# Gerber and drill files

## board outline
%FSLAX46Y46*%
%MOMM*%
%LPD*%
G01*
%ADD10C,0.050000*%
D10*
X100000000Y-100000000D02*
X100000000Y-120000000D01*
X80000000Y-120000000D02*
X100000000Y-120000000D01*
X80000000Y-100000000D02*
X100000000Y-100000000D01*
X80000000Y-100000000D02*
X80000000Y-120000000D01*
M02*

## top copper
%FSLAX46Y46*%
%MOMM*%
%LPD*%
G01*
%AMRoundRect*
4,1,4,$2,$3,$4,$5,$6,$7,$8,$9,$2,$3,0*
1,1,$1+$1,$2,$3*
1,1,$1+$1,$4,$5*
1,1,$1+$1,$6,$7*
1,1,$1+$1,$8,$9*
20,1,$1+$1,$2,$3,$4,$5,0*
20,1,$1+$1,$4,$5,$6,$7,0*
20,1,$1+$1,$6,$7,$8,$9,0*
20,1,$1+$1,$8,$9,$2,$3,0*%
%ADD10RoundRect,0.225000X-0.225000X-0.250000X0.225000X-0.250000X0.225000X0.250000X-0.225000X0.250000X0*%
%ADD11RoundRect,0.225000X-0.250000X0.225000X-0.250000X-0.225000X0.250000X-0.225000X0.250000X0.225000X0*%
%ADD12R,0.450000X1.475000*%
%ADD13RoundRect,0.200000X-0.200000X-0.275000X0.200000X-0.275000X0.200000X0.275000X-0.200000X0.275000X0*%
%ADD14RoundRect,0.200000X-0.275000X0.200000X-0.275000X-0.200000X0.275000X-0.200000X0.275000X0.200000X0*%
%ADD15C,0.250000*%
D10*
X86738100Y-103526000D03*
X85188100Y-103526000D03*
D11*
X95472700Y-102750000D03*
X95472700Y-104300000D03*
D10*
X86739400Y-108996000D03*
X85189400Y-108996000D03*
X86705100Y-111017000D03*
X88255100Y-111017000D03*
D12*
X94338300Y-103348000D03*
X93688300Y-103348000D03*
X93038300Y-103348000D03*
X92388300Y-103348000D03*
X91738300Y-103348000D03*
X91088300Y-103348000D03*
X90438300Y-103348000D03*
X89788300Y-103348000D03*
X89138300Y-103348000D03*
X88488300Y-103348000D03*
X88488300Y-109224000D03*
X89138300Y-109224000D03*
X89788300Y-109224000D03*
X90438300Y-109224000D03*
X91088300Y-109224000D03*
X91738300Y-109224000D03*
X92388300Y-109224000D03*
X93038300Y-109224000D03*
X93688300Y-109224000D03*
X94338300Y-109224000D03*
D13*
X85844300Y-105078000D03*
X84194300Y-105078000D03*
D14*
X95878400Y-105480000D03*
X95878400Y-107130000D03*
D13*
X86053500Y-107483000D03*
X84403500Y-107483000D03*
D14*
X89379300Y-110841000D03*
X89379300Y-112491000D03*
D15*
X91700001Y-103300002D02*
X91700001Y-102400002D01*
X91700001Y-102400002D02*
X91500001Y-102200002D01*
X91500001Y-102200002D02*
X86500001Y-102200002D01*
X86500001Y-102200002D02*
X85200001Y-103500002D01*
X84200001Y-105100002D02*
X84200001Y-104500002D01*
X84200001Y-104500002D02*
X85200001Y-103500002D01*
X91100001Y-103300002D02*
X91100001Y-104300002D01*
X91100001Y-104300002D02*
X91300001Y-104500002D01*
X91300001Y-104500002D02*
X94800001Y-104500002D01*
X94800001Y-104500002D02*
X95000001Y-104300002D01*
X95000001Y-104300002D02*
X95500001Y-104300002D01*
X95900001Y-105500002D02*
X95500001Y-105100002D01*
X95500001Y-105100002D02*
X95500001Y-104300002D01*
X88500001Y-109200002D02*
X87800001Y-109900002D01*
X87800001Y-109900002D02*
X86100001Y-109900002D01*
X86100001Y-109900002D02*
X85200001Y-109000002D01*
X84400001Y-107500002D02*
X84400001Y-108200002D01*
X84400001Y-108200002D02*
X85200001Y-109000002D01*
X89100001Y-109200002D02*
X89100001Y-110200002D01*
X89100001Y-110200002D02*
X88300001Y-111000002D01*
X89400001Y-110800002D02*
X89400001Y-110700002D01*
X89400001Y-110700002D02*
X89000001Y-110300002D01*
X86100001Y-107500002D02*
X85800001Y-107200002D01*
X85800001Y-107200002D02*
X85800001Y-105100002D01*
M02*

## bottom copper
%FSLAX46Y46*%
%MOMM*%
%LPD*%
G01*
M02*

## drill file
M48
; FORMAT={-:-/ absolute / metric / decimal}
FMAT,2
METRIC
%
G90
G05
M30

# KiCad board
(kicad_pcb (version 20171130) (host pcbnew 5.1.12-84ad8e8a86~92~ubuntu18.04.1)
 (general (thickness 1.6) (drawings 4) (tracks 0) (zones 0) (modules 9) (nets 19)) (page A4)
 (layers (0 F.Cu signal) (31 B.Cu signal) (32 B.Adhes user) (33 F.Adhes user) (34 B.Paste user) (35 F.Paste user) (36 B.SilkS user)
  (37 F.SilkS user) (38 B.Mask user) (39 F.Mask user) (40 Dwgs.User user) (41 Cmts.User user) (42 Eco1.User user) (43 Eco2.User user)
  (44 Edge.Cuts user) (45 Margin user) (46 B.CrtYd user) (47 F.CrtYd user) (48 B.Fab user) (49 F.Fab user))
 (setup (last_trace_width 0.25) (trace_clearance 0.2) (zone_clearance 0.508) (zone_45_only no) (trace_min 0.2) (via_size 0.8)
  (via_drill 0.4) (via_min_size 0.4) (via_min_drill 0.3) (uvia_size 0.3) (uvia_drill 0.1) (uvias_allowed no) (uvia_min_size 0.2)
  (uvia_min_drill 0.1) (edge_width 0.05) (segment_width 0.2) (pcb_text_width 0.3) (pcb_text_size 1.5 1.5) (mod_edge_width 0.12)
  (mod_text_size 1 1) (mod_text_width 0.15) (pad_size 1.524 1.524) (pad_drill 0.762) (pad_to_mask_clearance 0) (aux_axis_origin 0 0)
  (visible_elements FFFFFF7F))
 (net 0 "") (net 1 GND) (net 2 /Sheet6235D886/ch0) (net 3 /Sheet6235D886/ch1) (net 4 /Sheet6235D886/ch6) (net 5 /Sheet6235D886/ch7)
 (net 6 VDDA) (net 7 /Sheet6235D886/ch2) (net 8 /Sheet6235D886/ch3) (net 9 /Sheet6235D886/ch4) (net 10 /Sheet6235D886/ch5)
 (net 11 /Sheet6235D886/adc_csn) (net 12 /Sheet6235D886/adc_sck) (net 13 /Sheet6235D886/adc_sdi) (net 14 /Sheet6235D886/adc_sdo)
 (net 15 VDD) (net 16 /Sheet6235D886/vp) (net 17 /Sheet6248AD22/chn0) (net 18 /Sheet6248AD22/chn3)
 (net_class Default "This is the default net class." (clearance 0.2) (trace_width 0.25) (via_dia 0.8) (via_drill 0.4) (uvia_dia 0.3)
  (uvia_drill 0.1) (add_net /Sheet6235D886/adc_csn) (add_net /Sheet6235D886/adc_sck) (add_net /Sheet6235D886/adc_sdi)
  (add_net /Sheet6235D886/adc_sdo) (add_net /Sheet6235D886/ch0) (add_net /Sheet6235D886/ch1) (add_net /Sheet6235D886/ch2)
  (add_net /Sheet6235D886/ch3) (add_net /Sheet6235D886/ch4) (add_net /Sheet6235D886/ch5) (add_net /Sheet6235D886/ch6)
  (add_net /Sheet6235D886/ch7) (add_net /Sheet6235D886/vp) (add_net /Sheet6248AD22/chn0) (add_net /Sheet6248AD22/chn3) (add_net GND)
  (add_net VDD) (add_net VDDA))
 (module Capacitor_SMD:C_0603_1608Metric (layer F.Cu) (at 85.963100 103.526000)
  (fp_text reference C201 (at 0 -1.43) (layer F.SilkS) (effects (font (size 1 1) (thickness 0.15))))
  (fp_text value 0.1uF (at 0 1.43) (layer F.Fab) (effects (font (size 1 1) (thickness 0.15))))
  (pad 2 smd roundrect (at 0.775 0) (size 0.9 0.95) (layers F.Cu F.Mask F.Paste) (roundrect_rratio 0.25) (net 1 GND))
  (pad 1 smd roundrect (at -0.775 0) (size 0.9 0.95) (layers F.Cu F.Mask F.Paste) (roundrect_rratio 0.25) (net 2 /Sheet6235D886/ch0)))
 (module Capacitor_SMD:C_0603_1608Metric (layer F.Cu) (at 95.472700 103.525000 270.000000)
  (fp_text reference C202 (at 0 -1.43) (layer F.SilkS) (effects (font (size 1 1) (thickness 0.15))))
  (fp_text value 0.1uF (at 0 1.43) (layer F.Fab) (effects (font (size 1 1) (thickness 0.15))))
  (pad 1 smd roundrect (at -0.775 0 270.000000) (size 0.9 0.95) (layers F.Cu F.Mask F.Paste) (roundrect_rratio 0.25) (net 1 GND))
  (pad 2 smd roundrect (at 0.775 0 270.000000) (size 0.9 0.95) (layers F.Cu F.Mask F.Paste) (roundrect_rratio 0.25)
   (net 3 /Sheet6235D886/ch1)))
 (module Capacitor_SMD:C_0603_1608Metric (layer F.Cu) (at 85.964400 108.996000)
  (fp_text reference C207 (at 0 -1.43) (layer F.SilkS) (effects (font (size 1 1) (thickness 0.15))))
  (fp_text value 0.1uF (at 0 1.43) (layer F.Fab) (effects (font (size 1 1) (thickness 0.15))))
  (pad 2 smd roundrect (at 0.775 0) (size 0.9 0.95) (layers F.Cu F.Mask F.Paste) (roundrect_rratio 0.25) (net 1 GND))
  (pad 1 smd roundrect (at -0.775 0) (size 0.9 0.95) (layers F.Cu F.Mask F.Paste) (roundrect_rratio 0.25) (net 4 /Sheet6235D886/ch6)))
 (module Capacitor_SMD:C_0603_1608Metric (layer F.Cu) (at 87.480100 111.017000)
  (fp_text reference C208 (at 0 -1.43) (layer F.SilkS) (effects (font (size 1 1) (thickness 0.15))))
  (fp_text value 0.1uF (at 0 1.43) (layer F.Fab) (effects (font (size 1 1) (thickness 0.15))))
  (pad 1 smd roundrect (at -0.775 0) (size 0.9 0.95) (layers F.Cu F.Mask F.Paste) (roundrect_rratio 0.25) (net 1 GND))
  (pad 2 smd roundrect (at 0.775 0) (size 0.9 0.95) (layers F.Cu F.Mask F.Paste) (roundrect_rratio 0.25) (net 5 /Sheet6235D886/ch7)))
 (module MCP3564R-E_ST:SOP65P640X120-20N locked (layer F.Cu) (at 91.413300 106.286000 270.000000)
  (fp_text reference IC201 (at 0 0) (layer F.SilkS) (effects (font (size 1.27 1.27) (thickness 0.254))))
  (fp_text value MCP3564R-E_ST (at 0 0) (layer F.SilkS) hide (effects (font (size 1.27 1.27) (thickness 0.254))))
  (pad 1 smd rect (at -2.938 -2.925) (size 0.45 1.475) (layers F.Cu F.Mask F.Paste) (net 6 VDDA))
  (pad 2 smd rect (at -2.938 -2.275) (size 0.45 1.475) (layers F.Cu F.Mask F.Paste) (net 1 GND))
  (pad 3 smd rect (at -2.938 -1.625) (size 0.45 1.475) (layers F.Cu F.Mask F.Paste) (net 1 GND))
  (pad 4 smd rect (at -2.938 -0.975) (size 0.45 1.475) (layers F.Cu F.Mask F.Paste))
  (pad 5 smd rect (at -2.938 -0.325) (size 0.45 1.475) (layers F.Cu F.Mask F.Paste) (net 2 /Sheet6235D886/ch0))
  (pad 6 smd rect (at -2.938 0.325) (size 0.45 1.475) (layers F.Cu F.Mask F.Paste) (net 3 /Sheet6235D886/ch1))
  (pad 7 smd rect (at -2.938 0.975) (size 0.45 1.475) (layers F.Cu F.Mask F.Paste) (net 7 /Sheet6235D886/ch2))
  (pad 8 smd rect (at -2.938 1.625) (size 0.45 1.475) (layers F.Cu F.Mask F.Paste) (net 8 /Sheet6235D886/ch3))
  (pad 9 smd rect (at -2.938 2.275) (size 0.45 1.475) (layers F.Cu F.Mask F.Paste) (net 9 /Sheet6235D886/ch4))
  (pad 10 smd rect (at -2.938 2.925) (size 0.45 1.475) (layers F.Cu F.Mask F.Paste) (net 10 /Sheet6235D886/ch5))
  (pad 11 smd rect (at 2.938 2.925) (size 0.45 1.475) (layers F.Cu F.Mask F.Paste) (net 4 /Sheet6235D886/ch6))
  (pad 12 smd rect (at 2.938 2.275) (size 0.45 1.475) (layers F.Cu F.Mask F.Paste) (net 5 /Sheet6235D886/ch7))
  (pad 13 smd rect (at 2.938 1.625) (size 0.45 1.475) (layers F.Cu F.Mask F.Paste) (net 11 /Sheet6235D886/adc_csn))
  (pad 14 smd rect (at 2.938 0.975) (size 0.45 1.475) (layers F.Cu F.Mask F.Paste) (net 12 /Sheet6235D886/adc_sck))
  (pad 15 smd rect (at 2.938 0.325) (size 0.45 1.475) (layers F.Cu F.Mask F.Paste) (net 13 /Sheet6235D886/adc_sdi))
  (pad 16 smd rect (at 2.938 -0.325) (size 0.45 1.475) (layers F.Cu F.Mask F.Paste) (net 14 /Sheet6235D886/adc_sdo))
  (pad 17 smd rect (at 2.938 -0.975) (size 0.45 1.475) (layers F.Cu F.Mask F.Paste))
  (pad 18 smd rect (at 2.938 -1.625) (size 0.45 1.475) (layers F.Cu F.Mask F.Paste))
  (pad 19 smd rect (at 2.938 -2.275) (size 0.45 1.475) (layers F.Cu F.Mask F.Paste) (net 1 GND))
  (pad 20 smd rect (at 2.938 -2.925) (size 0.45 1.475) (layers F.Cu F.Mask F.Paste) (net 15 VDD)))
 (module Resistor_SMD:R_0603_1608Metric (layer F.Cu) (at 85.019300 105.078000)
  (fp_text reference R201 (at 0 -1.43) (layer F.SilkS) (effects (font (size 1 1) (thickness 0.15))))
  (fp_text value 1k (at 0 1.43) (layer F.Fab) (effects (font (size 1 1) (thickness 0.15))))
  (pad 2 smd roundrect (at 0.825 0) (size 0.8 0.95) (layers F.Cu F.Mask F.Paste) (roundrect_rratio 0.25) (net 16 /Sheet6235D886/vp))
  (pad 1 smd roundrect (at -0.825 0) (size 0.8 0.95) (layers F.Cu F.Mask F.Paste) (roundrect_rratio 0.25) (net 2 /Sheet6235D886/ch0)))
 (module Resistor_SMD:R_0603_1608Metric (layer F.Cu) (at 95.878400 106.305000 270.000000)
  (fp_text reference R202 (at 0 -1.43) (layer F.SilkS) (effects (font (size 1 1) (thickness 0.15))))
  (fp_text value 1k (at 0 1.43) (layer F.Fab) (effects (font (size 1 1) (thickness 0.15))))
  (pad 1 smd roundrect (at -0.825 0 270.000000) (size 0.8 0.95) (layers F.Cu F.Mask F.Paste) (roundrect_rratio 0.25)
   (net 3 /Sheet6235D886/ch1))
  (pad 2 smd roundrect (at 0.825 0 270.000000) (size 0.8 0.95) (layers F.Cu F.Mask F.Paste) (roundrect_rratio 0.25)
   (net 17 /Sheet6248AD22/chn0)))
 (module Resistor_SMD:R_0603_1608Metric (layer F.Cu) (at 85.228500 107.483000)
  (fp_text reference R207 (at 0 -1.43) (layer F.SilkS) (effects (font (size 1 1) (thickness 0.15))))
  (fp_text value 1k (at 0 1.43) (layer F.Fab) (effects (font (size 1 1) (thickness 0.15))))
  (pad 2 smd roundrect (at 0.825 0) (size 0.8 0.95) (layers F.Cu F.Mask F.Paste) (roundrect_rratio 0.25) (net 16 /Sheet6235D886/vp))
  (pad 1 smd roundrect (at -0.825 0) (size 0.8 0.95) (layers F.Cu F.Mask F.Paste) (roundrect_rratio 0.25) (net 4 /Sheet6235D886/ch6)))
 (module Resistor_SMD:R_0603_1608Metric (layer F.Cu) (at 89.379300 111.666000 270.000000)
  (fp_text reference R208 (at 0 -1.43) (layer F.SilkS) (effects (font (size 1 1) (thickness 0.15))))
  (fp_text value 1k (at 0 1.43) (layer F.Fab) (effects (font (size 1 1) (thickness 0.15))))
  (pad 1 smd roundrect (at -0.825 0 270.000000) (size 0.8 0.95) (layers F.Cu F.Mask F.Paste) (roundrect_rratio 0.25)
   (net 5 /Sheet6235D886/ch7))
  (pad 2 smd roundrect (at 0.825 0 270.000000) (size 0.8 0.95) (layers F.Cu F.Mask F.Paste) (roundrect_rratio 0.25)
   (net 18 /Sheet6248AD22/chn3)))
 (gr_line (start 100 100) (end 100 120) (layer Edge.Cuts) (width 0.05))
 (gr_line (start 80 120) (end 100 120) (layer Edge.Cuts) (width 0.05))
 (gr_line (start 80 100) (end 100 100) (layer Edge.Cuts) (width 0.05))
 (gr_line (start 80 100) (end 80 120) (layer Edge.Cuts) (width 0.05))
 (segment (start 91.700001 103.300002) (end 91.700001 102.400002) (width 0.250000) (layer F.Cu) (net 2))
 (segment (start 91.700001 102.400002) (end 91.500001 102.200002) (width 0.250000) (layer F.Cu) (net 2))
 (segment (start 91.500001 102.200002) (end 86.500001 102.200002) (width 0.250000) (layer F.Cu) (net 2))
 (segment (start 86.500001 102.200002) (end 85.200001 103.500002) (width 0.250000) (layer F.Cu) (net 2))
 (segment (start 84.200001 105.100002) (end 84.200001 104.500002) (width 0.250000) (layer F.Cu) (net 2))
 (segment (start 84.200001 104.500002) (end 85.200001 103.500002) (width 0.250000) (layer F.Cu) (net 2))
 (segment (start 91.100001 103.300002) (end 91.100001 104.300002) (width 0.250000) (layer F.Cu) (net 3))
 (segment (start 91.100001 104.300002) (end 91.300001 104.500002) (width 0.250000) (layer F.Cu) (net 3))
 (segment (start 91.300001 104.500002) (end 94.800001 104.500002) (width 0.250000) (layer F.Cu) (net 3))
 (segment (start 94.800001 104.500002) (end 95.000001 104.300002) (width 0.250000) (layer F.Cu) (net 3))
 (segment (start 95.000001 104.300002) (end 95.500001 104.300002) (width 0.250000) (layer F.Cu) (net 3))
 (segment (start 95.900001 105.500002) (end 95.500001 105.100002) (width 0.250000) (layer F.Cu) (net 3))
 (segment (start 95.500001 105.100002) (end 95.500001 104.300002) (width 0.250000) (layer F.Cu) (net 3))
 (segment (start 88.500001 109.200002) (end 87.800001 109.900002) (width 0.250000) (layer F.Cu) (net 4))
 (segment (start 87.800001 109.900002) (end 86.100001 109.900002) (width 0.250000) (layer F.Cu) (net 4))
 (segment (start 86.100001 109.900002) (end 85.200001 109.000002) (width 0.250000) (layer F.Cu) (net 4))
 (segment (start 84.400001 107.500002) (end 84.400001 108.200002) (width 0.250000) (layer F.Cu) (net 4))
 (segment (start 84.400001 108.200002) (end 85.200001 109.000002) (width 0.250000) (layer F.Cu) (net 4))
 (segment (start 89.100001 109.200002) (end 89.100001 110.200002) (width 0.250000) (layer F.Cu) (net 5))
 (segment (start 89.100001 110.200002) (end 88.300001 111.000002) (width 0.250000) (layer F.Cu) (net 5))
 (segment (start 89.400001 110.800002) (end 89.400001 110.700002) (width 0.250000) (layer F.Cu) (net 5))
 (segment (start 89.400001 110.700002) (end 89.000001 110.300002) (width 0.250000) (layer F.Cu) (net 5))
 (segment (start 86.100001 107.500002) (end 85.800001 107.200002) (width 0.250000) (layer F.Cu) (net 16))
 (segment (start 85.800001 107.200002) (end 85.800001 105.100002) (width 0.250000) (layer F.Cu) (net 16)))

